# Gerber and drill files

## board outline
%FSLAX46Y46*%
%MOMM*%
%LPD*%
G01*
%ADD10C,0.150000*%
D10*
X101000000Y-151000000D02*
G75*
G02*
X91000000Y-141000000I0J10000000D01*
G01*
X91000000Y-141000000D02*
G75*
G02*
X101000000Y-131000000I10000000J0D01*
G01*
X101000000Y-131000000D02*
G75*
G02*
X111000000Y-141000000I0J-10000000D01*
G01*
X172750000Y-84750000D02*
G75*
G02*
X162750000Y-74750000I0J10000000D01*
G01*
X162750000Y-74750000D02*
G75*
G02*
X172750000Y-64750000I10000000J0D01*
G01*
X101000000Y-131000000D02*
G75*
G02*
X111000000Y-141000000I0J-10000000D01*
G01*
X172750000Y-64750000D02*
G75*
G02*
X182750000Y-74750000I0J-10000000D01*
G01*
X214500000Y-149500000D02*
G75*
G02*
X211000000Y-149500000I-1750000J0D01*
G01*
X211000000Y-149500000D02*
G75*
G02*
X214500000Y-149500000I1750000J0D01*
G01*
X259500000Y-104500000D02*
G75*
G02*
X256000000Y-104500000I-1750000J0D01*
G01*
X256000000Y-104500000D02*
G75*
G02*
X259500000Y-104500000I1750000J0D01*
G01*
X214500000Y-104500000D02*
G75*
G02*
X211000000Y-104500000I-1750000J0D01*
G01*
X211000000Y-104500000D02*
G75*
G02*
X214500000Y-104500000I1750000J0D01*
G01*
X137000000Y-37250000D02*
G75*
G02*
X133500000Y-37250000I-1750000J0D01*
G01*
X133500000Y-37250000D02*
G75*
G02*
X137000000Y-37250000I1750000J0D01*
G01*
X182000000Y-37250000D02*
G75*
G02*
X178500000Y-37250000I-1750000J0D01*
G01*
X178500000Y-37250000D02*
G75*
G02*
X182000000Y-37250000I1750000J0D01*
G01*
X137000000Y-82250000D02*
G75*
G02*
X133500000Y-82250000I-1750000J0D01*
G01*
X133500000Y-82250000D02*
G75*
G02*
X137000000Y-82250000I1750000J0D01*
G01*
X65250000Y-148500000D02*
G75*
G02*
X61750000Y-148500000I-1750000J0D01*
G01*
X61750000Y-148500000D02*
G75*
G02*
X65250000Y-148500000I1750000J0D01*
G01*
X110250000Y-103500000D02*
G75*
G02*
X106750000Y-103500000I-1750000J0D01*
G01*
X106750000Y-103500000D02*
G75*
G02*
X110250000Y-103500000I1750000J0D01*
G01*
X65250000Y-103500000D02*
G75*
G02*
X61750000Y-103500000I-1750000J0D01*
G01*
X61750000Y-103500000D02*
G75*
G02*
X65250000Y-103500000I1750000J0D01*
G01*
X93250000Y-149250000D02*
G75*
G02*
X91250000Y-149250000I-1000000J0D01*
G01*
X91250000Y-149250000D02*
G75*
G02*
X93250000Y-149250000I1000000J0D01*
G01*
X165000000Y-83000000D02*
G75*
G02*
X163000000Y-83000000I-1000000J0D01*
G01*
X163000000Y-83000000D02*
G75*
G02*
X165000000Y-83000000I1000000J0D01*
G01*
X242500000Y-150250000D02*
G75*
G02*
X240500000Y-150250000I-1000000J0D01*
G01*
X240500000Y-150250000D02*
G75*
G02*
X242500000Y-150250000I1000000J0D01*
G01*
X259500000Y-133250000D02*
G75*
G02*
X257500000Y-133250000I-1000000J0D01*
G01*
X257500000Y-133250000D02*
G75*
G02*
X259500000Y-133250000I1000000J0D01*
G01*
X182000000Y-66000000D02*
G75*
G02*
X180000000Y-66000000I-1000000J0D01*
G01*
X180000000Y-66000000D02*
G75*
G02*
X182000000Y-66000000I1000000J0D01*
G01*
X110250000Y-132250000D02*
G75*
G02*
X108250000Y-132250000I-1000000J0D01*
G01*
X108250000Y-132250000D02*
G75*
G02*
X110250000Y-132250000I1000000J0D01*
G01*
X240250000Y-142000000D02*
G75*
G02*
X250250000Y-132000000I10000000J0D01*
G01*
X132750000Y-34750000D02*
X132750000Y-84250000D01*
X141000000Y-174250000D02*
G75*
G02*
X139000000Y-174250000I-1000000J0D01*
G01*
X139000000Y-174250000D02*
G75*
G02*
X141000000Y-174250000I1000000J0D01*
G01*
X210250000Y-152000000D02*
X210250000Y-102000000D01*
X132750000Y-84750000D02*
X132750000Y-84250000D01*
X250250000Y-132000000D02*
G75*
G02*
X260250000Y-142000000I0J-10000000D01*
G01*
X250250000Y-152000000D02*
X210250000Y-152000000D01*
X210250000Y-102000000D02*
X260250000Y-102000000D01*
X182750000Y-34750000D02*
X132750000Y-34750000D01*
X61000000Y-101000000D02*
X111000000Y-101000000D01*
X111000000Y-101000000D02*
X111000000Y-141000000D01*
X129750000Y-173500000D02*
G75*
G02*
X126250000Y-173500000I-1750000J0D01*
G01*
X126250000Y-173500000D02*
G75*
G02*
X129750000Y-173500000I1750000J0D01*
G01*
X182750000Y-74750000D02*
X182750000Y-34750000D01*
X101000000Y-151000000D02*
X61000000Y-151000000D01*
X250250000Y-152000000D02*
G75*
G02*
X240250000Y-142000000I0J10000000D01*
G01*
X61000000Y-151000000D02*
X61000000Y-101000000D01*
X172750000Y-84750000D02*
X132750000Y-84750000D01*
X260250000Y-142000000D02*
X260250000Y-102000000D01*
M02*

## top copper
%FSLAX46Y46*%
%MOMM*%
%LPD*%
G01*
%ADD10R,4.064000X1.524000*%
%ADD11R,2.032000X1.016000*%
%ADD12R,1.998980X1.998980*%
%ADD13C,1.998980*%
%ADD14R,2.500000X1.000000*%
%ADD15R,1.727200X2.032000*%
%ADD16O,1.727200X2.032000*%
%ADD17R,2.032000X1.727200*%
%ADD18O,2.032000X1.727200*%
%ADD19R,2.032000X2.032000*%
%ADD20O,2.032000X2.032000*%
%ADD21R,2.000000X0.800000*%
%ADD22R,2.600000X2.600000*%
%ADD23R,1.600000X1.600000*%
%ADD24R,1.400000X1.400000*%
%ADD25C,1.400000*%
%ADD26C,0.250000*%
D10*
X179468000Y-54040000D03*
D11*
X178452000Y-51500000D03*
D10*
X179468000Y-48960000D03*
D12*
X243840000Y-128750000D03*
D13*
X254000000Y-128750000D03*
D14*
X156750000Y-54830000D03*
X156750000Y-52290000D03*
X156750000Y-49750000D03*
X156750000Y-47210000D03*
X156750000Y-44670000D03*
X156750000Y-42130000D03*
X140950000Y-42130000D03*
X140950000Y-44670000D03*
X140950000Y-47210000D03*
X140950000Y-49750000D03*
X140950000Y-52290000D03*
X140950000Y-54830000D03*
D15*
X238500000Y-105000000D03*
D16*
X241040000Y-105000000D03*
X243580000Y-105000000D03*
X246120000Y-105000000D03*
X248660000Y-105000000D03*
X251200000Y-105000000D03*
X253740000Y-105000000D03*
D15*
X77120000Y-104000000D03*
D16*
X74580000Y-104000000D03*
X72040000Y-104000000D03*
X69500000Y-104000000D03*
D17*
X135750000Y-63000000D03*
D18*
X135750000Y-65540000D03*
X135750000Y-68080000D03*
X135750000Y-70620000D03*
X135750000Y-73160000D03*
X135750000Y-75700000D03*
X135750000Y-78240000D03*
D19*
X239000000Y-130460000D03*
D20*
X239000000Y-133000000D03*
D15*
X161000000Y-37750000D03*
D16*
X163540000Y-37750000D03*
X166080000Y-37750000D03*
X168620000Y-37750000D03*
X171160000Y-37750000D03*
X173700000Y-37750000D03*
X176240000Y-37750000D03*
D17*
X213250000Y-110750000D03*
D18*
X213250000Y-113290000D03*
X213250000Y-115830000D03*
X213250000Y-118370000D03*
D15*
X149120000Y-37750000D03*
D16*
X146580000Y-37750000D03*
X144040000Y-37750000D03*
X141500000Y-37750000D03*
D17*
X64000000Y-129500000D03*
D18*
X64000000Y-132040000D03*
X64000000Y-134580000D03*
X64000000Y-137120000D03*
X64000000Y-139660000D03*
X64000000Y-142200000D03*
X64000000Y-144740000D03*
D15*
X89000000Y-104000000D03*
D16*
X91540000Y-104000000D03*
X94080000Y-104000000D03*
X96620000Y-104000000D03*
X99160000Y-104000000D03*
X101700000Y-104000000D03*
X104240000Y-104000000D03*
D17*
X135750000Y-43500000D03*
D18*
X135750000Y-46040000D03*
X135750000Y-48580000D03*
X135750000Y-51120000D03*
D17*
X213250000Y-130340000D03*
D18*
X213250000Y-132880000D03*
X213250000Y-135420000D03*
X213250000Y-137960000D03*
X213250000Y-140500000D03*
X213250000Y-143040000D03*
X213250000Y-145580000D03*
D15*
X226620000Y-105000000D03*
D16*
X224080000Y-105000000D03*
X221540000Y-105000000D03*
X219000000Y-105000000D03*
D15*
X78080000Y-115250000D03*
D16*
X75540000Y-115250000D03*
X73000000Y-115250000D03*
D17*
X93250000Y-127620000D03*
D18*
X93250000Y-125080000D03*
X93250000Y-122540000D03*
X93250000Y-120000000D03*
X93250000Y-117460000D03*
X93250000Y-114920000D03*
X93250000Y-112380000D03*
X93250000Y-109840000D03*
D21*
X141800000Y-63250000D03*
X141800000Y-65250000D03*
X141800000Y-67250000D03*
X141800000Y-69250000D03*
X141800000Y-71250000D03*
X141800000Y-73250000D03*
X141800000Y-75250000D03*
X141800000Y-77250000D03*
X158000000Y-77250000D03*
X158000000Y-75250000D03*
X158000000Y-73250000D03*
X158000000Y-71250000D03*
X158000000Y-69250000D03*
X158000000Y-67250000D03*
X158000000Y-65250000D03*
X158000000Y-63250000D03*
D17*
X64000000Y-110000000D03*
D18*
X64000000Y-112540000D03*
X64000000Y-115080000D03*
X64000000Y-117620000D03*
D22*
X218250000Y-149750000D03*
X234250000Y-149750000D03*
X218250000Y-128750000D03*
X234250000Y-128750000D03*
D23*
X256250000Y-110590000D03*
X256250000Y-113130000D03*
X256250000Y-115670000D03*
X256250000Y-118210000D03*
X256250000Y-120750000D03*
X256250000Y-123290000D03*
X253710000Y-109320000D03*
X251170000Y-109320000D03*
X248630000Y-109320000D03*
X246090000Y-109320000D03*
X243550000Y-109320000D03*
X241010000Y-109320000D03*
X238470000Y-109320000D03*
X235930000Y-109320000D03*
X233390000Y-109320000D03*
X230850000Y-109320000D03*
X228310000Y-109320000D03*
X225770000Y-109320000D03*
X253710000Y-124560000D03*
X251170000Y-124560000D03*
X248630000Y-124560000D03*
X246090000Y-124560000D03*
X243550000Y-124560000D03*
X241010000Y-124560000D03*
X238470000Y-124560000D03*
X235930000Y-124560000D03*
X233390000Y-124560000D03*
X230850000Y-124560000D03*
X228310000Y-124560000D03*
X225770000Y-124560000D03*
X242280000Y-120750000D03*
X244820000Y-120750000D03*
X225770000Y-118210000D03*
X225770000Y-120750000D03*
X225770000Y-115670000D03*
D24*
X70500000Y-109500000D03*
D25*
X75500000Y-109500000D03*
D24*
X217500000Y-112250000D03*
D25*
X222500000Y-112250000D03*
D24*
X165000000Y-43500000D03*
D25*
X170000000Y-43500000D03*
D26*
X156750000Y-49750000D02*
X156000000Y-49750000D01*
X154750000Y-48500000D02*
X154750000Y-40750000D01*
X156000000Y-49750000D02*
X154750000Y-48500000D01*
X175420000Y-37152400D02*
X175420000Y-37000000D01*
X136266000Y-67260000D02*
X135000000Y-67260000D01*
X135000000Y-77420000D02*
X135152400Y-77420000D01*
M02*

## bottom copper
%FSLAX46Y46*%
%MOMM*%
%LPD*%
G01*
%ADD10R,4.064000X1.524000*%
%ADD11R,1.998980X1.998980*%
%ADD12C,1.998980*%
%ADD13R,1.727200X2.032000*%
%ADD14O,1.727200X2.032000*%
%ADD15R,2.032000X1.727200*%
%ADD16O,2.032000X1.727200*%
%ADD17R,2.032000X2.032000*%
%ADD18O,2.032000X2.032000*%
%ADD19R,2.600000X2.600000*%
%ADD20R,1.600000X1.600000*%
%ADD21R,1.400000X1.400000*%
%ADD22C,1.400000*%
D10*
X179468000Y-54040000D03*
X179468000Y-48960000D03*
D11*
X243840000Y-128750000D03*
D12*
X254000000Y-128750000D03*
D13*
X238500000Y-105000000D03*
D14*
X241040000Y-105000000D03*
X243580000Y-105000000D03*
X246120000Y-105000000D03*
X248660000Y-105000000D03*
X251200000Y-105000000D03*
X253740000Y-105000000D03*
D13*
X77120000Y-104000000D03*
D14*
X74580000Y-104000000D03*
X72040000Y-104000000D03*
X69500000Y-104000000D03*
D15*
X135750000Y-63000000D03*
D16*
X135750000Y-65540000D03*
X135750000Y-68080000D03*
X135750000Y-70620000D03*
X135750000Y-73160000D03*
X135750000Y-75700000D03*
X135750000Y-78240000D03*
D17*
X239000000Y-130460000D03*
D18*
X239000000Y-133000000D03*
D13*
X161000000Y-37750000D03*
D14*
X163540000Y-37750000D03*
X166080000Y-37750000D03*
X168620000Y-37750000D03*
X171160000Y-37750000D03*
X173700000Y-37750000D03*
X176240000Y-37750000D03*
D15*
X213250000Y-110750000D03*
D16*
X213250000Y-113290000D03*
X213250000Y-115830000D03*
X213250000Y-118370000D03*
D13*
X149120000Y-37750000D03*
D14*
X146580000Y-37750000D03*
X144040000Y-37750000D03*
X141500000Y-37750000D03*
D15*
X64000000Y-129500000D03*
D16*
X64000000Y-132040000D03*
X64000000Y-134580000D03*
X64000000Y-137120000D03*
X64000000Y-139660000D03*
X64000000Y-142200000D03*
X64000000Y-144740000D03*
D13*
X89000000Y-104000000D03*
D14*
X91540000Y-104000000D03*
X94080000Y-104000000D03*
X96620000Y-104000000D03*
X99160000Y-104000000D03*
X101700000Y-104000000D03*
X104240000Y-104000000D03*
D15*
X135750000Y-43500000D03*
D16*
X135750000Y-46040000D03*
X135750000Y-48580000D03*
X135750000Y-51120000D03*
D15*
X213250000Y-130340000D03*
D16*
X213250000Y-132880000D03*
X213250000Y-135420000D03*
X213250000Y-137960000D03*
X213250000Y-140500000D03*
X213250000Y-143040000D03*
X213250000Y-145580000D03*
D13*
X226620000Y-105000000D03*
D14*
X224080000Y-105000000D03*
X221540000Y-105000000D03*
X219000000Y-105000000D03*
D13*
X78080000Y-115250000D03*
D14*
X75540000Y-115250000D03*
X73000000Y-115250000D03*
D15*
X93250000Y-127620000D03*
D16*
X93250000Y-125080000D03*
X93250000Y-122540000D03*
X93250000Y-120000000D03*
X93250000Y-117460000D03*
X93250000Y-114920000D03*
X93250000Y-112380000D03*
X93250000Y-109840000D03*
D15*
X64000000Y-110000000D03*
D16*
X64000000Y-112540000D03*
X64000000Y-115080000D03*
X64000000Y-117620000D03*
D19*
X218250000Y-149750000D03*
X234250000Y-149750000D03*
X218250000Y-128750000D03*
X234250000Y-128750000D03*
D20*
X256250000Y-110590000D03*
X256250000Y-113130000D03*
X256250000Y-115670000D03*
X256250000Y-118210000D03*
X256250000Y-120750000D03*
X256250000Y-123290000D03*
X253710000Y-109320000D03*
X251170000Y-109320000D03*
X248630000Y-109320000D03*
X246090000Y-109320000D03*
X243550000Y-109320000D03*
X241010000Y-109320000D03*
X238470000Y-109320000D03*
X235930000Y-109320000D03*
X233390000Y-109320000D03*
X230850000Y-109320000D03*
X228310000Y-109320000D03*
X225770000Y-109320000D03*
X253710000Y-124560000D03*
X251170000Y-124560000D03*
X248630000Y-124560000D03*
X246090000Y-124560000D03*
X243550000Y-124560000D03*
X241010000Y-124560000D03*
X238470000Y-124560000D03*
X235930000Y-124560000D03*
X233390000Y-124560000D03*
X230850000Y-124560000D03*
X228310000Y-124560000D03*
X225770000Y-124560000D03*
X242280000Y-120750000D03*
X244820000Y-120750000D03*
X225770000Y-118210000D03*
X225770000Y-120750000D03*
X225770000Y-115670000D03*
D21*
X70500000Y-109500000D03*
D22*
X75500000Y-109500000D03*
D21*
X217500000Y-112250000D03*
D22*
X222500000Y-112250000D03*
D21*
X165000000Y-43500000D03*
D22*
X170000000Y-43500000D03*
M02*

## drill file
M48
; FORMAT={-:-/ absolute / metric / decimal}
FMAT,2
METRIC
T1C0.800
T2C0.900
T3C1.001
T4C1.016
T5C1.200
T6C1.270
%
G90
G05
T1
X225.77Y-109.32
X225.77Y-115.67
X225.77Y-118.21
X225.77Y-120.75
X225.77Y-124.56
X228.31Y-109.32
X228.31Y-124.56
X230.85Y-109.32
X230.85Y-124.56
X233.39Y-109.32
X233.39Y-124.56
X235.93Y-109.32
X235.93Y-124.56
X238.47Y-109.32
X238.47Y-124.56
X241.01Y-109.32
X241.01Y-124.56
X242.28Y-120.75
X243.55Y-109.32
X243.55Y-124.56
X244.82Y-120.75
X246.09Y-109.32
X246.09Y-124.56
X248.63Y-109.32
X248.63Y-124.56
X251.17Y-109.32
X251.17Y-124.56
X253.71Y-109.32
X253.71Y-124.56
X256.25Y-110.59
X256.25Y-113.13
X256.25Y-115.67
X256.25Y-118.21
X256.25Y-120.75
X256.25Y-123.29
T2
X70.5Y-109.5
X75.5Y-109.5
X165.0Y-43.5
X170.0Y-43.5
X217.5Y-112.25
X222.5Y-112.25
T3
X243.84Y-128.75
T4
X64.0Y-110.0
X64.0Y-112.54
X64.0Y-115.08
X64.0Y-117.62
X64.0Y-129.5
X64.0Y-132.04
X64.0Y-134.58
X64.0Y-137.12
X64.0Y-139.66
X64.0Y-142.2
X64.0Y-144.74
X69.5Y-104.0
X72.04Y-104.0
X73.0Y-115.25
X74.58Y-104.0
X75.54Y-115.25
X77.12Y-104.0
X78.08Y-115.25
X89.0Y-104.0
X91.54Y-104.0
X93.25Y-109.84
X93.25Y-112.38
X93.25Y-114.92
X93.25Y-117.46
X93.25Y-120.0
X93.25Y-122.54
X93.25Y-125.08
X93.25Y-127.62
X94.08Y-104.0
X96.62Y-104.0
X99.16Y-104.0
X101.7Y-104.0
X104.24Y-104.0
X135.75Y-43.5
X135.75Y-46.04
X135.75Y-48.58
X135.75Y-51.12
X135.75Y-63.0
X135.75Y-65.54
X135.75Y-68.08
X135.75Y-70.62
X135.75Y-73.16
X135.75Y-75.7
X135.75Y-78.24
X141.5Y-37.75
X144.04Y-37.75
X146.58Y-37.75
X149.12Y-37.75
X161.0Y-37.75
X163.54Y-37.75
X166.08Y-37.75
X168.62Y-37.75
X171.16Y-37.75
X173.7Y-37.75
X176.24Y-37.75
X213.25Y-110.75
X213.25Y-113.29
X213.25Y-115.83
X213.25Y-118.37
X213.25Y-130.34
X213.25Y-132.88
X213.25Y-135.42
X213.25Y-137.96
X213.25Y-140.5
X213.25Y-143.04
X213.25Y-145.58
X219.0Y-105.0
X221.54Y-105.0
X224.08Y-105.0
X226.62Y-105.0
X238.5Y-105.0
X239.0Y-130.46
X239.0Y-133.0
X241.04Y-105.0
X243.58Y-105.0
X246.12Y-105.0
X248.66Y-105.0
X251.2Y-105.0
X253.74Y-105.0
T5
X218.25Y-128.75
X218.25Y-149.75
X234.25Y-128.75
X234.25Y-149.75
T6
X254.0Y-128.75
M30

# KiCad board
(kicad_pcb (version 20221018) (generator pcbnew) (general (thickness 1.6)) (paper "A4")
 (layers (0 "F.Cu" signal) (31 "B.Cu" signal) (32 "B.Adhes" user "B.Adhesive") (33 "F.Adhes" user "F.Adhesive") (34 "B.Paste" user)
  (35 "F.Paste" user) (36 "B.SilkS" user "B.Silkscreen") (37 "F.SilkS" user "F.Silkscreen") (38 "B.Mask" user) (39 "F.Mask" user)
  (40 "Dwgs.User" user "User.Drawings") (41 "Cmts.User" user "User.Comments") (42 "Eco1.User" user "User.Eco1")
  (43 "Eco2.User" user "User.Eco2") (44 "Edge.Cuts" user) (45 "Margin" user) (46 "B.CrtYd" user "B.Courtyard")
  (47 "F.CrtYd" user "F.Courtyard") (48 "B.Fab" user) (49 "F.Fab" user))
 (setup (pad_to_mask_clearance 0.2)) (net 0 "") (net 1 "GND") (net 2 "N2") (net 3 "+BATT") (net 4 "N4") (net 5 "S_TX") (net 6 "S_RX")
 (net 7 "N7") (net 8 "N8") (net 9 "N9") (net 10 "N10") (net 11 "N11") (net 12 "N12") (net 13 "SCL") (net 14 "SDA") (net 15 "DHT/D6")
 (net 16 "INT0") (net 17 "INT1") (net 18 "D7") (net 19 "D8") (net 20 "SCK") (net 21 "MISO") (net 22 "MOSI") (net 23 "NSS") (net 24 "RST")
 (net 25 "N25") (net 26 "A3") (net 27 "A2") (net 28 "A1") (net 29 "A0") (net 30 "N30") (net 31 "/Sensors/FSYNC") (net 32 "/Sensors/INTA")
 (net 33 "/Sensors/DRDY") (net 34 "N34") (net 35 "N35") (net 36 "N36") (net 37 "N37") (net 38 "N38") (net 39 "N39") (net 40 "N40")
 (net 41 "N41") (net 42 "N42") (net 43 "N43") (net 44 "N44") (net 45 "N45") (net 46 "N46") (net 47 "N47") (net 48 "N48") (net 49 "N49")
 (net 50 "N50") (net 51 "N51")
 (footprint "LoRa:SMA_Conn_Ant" (layer "F.Cu") (at 181.5 51.5 180)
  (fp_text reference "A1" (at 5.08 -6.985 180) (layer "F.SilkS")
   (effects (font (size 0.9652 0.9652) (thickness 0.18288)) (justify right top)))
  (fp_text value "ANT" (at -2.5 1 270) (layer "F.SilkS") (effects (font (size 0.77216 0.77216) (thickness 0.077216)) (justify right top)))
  (pad "" smd rect (at 2.032 -2.54 270) (size 1.524 4.064) (layers "B.Cu" "B.Paste" "B.Mask"))
  (pad "" smd rect (at 2.032 2.54 270) (size 1.524 4.064) (layers "B.Cu" "B.Paste" "B.Mask"))
  (pad "1" smd rect (at 2.032 -2.54 270) (size 1.524 4.064) (layers "F.Cu" "F.Paste" "F.Mask") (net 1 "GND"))
  (pad "2" smd rect (at 3.048 0 270) (size 1.016 2.032) (layers "F.Cu" "F.Paste" "F.Mask") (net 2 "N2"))
  (pad "3" smd rect (at 2.032 2.54 270) (size 1.524 4.064) (layers "F.Cu" "F.Paste" "F.Mask") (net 1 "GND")))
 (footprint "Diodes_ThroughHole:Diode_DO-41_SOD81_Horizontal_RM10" (layer "F.Cu") (at 243.84 128.75254)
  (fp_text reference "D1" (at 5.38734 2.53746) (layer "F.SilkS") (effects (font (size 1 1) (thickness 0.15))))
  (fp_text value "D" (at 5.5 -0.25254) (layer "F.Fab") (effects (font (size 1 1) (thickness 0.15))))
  (pad "1" thru_hole rect (at 0 -0.00254 180) (size 1.99898 1.99898) (drill 1.00076) (layers "*.Cu" "*.Mask" "F.SilkS") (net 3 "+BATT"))
  (pad "2" thru_hole circle (at 10.16 -0.00254 180) (size 1.99898 1.99898) (drill 1.27) (layers "*.Cu" "*.Mask" "F.SilkS") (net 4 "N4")))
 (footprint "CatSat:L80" (layer "F.Cu") (at 148.883668 49.118506 180) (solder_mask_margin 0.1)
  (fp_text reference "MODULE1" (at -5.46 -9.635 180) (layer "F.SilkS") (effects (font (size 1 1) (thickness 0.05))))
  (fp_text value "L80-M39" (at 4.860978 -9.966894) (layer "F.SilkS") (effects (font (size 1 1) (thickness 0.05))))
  (pad "1" smd rect (at -7.866332 -5.711494) (size 2.5 1) (layers "F.Cu" "F.Paste" "F.Mask") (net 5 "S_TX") (solder_mask_margin 0.2))
  (pad "2" smd rect (at -7.866332 -3.171494) (size 2.5 1) (layers "F.Cu" "F.Paste" "F.Mask") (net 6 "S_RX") (solder_mask_margin 0.2))
  (pad "3" smd rect (at -7.866332 -0.631494) (size 2.5 1) (layers "F.Cu" "F.Paste" "F.Mask") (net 1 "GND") (solder_mask_margin 0.2))
  (pad "4" smd rect (at -7.866332 1.908506) (size 2.5 1) (layers "F.Cu" "F.Paste" "F.Mask") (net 3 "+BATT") (solder_mask_margin 0.2))
  (pad "5" smd rect (at -7.866332 4.448506) (size 2.5 1) (layers "F.Cu" "F.Paste" "F.Mask") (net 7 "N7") (solder_mask_margin 0.2))
  (pad "6" smd rect (at -7.866332 6.988506) (size 2.5 1) (layers "F.Cu" "F.Paste" "F.Mask") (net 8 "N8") (solder_mask_margin 0.2))
  (pad "7" smd rect (at 7.933668 6.988506 180) (size 2.5 1) (layers "F.Cu" "F.Paste" "F.Mask") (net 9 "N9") (solder_mask_margin 0.2))
  (pad "8" smd rect (at 7.933668 4.448506 180) (size 2.5 1) (layers "F.Cu" "F.Paste" "F.Mask") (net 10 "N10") (solder_mask_margin 0.2))
  (pad "9" smd rect (at 7.933668 1.908506 180) (size 2.5 1) (layers "F.Cu" "F.Paste" "F.Mask") (solder_mask_margin 0.2))
  (pad "10" smd rect (at 7.933668 -0.631494 180) (size 2.5 1) (layers "F.Cu" "F.Paste" "F.Mask") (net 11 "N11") (solder_mask_margin 0.2))
  (pad "11" smd rect (at 7.933668 -3.171494 180) (size 2.5 1) (layers "F.Cu" "F.Paste" "F.Mask") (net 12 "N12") (solder_mask_margin 0.2))
  (pad "12" smd rect (at 7.933668 -5.711494) (size 2.5 1) (layers "F.Cu" "F.Paste" "F.Mask") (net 1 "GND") (solder_mask_margin 0.2)))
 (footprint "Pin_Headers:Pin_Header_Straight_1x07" (layer "F.Cu") (at 238.5 105 90)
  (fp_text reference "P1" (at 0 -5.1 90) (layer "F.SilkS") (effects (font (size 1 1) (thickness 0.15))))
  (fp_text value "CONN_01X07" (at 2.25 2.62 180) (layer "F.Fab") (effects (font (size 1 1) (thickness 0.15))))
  (pad "1" thru_hole rect (at 0 0 90) (size 2.032 1.7272) (drill 1.016) (layers "*.Cu" "*.Mask" "F.SilkS") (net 1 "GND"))
  (pad "2" thru_hole oval (at 0 2.54 90) (size 2.032 1.7272) (drill 1.016) (layers "*.Cu" "*.Mask" "F.SilkS") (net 3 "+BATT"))
  (pad "3" thru_hole oval (at 0 5.08 90) (size 2.032 1.7272) (drill 1.016) (layers "*.Cu" "*.Mask" "F.SilkS") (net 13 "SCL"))
  (pad "4" thru_hole oval (at 0 7.62 90) (size 2.032 1.7272) (drill 1.016) (layers "*.Cu" "*.Mask" "F.SilkS") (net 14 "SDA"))
  (pad "5" thru_hole oval (at 0 10.16 90) (size 2.032 1.7272) (drill 1.016) (layers "*.Cu" "*.Mask" "F.SilkS") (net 6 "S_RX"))
  (pad "6" thru_hole oval (at 0 12.7 90) (size 2.032 1.7272) (drill 1.016) (layers "*.Cu" "*.Mask" "F.SilkS") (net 5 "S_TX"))
  (pad "7" thru_hole oval (at 0 15.24 90) (size 2.032 1.7272) (drill 1.016) (layers "*.Cu" "*.Mask" "F.SilkS") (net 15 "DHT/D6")))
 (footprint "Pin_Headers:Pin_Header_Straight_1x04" (layer "F.Cu") (at 77.12 104 -90)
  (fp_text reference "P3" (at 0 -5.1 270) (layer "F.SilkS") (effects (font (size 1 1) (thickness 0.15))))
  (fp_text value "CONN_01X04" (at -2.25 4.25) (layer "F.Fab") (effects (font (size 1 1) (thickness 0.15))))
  (pad "1" thru_hole rect (at 0 0 270) (size 2.032 1.7272) (drill 1.016) (layers "*.Cu" "*.Mask" "F.SilkS") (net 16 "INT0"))
  (pad "2" thru_hole oval (at 0 2.54 270) (size 2.032 1.7272) (drill 1.016) (layers "*.Cu" "*.Mask" "F.SilkS") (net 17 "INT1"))
  (pad "3" thru_hole oval (at 0 5.08 270) (size 2.032 1.7272) (drill 1.016) (layers "*.Cu" "*.Mask" "F.SilkS") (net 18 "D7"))
  (pad "4" thru_hole oval (at 0 7.62 270) (size 2.032 1.7272) (drill 1.016) (layers "*.Cu" "*.Mask" "F.SilkS") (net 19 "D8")))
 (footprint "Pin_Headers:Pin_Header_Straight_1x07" (layer "F.Cu") (at 135.75 63)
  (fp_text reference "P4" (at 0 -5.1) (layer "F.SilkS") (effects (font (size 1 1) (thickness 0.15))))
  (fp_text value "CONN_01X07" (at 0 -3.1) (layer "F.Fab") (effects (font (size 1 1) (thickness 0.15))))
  (pad "1" thru_hole rect (at 0 0) (size 2.032 1.7272) (drill 1.016) (layers "*.Cu" "*.Mask" "F.SilkS") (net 3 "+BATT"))
  (pad "2" thru_hole oval (at 0 2.54) (size 2.032 1.7272) (drill 1.016) (layers "*.Cu" "*.Mask" "F.SilkS") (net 1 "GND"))
  (pad "3" thru_hole oval (at 0 5.08) (size 2.032 1.7272) (drill 1.016) (layers "*.Cu" "*.Mask" "F.SilkS") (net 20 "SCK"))
  (pad "4" thru_hole oval (at 0 7.62) (size 2.032 1.7272) (drill 1.016) (layers "*.Cu" "*.Mask" "F.SilkS") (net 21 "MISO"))
  (pad "5" thru_hole oval (at 0 10.16) (size 2.032 1.7272) (drill 1.016) (layers "*.Cu" "*.Mask" "F.SilkS") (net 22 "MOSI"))
  (pad "6" thru_hole oval (at 0 12.7) (size 2.032 1.7272) (drill 1.016) (layers "*.Cu" "*.Mask" "F.SilkS") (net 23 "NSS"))
  (pad "7" thru_hole oval (at 0 15.24) (size 2.032 1.7272) (drill 1.016) (layers "*.Cu" "*.Mask" "F.SilkS") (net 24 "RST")))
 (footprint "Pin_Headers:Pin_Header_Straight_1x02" (layer "F.Cu") (at 239 130.46)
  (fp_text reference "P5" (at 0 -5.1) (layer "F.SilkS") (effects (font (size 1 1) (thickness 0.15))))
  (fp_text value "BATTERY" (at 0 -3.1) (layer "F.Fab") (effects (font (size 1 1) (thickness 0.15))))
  (pad "1" thru_hole rect (at 0 0) (size 2.032 2.032) (drill 1.016) (layers "*.Cu" "*.Mask" "F.SilkS") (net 4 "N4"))
  (pad "2" thru_hole oval (at 0 2.54) (size 2.032 2.032) (drill 1.016) (layers "*.Cu" "*.Mask" "F.SilkS") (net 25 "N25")))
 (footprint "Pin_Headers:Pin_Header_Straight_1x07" (layer "F.Cu") (at 161 37.75 90)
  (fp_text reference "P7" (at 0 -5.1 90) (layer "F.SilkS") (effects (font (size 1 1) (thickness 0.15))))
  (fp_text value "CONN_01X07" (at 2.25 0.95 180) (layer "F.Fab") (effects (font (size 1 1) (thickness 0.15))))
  (pad "1" thru_hole rect (at 0 0 90) (size 2.032 1.7272) (drill 1.016) (layers "*.Cu" "*.Mask" "F.SilkS") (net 1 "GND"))
  (pad "2" thru_hole oval (at 0 2.54 90) (size 2.032 1.7272) (drill 1.016) (layers "*.Cu" "*.Mask" "F.SilkS") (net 3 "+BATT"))
  (pad "3" thru_hole oval (at 0 5.08 90) (size 2.032 1.7272) (drill 1.016) (layers "*.Cu" "*.Mask" "F.SilkS") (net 13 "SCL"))
  (pad "4" thru_hole oval (at 0 7.62 90) (size 2.032 1.7272) (drill 1.016) (layers "*.Cu" "*.Mask" "F.SilkS") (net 14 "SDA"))
  (pad "5" thru_hole oval (at 0 10.16 90) (size 2.032 1.7272) (drill 1.016) (layers "*.Cu" "*.Mask" "F.SilkS") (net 6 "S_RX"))
  (pad "6" thru_hole oval (at 0 12.7 90) (size 2.032 1.7272) (drill 1.016) (layers "*.Cu" "*.Mask" "F.SilkS") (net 5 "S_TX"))
  (pad "7" thru_hole oval (at 0 15.24 90) (size 2.032 1.7272) (drill 1.016) (layers "*.Cu" "*.Mask" "F.SilkS") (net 15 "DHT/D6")))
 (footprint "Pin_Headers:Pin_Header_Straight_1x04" (layer "F.Cu") (at 213.25 110.75)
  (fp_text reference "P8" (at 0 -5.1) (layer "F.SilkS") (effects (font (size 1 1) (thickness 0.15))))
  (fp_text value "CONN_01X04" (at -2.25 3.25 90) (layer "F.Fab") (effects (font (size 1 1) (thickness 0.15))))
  (pad "1" thru_hole rect (at 0 0) (size 2.032 1.7272) (drill 1.016) (layers "*.Cu" "*.Mask" "F.SilkS") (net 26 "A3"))
  (pad "2" thru_hole oval (at 0 2.54) (size 2.032 1.7272) (drill 1.016) (layers "*.Cu" "*.Mask" "F.SilkS") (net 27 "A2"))
  (pad "3" thru_hole oval (at 0 5.08) (size 2.032 1.7272) (drill 1.016) (layers "*.Cu" "*.Mask" "F.SilkS") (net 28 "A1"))
  (pad "4" thru_hole oval (at 0 7.62) (size 2.032 1.7272) (drill 1.016) (layers "*.Cu" "*.Mask" "F.SilkS") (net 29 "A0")))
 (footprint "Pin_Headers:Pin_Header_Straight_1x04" (layer "F.Cu") (at 149.12 37.75 -90)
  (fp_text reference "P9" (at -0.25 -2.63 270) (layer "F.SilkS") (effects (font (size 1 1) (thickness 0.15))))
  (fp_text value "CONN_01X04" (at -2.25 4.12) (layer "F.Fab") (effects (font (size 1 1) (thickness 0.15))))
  (pad "1" thru_hole rect (at 0 0 270) (size 2.032 1.7272) (drill 1.016) (layers "*.Cu" "*.Mask" "F.SilkS") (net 16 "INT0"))
  (pad "2" thru_hole oval (at 0 2.54 270) (size 2.032 1.7272) (drill 1.016) (layers "*.Cu" "*.Mask" "F.SilkS") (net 17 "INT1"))
  (pad "3" thru_hole oval (at 0 5.08 270) (size 2.032 1.7272) (drill 1.016) (layers "*.Cu" "*.Mask" "F.SilkS") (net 18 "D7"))
  (pad "4" thru_hole oval (at 0 7.62 270) (size 2.032 1.7272) (drill 1.016) (layers "*.Cu" "*.Mask" "F.SilkS") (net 19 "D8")))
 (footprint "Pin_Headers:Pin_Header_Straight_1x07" (layer "F.Cu") (at 64 129.5)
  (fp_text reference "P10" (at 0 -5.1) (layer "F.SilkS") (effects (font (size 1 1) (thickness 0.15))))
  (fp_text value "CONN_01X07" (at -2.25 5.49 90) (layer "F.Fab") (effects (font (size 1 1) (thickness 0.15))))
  (pad "1" thru_hole rect (at 0 0) (size 2.032 1.7272) (drill 1.016) (layers "*.Cu" "*.Mask" "F.SilkS") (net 3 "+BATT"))
  (pad "2" thru_hole oval (at 0 2.54) (size 2.032 1.7272) (drill 1.016) (layers "*.Cu" "*.Mask" "F.SilkS") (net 1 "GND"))
  (pad "3" thru_hole oval (at 0 5.08) (size 2.032 1.7272) (drill 1.016) (layers "*.Cu" "*.Mask" "F.SilkS") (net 20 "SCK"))
  (pad "4" thru_hole oval (at 0 7.62) (size 2.032 1.7272) (drill 1.016) (layers "*.Cu" "*.Mask" "F.SilkS") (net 21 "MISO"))
  (pad "5" thru_hole oval (at 0 10.16) (size 2.032 1.7272) (drill 1.016) (layers "*.Cu" "*.Mask" "F.SilkS") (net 22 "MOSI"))
  (pad "6" thru_hole oval (at 0 12.7) (size 2.032 1.7272) (drill 1.016) (layers "*.Cu" "*.Mask" "F.SilkS") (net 23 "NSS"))
  (pad "7" thru_hole oval (at 0 15.24) (size 2.032 1.7272) (drill 1.016) (layers "*.Cu" "*.Mask" "F.SilkS") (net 24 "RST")))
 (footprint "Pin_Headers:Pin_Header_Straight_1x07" (layer "F.Cu") (at 89 104 90)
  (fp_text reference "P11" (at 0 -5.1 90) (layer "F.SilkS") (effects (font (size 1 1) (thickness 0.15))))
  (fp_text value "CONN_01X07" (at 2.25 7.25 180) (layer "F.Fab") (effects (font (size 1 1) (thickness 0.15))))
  (pad "1" thru_hole rect (at 0 0 90) (size 2.032 1.7272) (drill 1.016) (layers "*.Cu" "*.Mask" "F.SilkS") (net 1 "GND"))
  (pad "2" thru_hole oval (at 0 2.54 90) (size 2.032 1.7272) (drill 1.016) (layers "*.Cu" "*.Mask" "F.SilkS") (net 3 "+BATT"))
  (pad "3" thru_hole oval (at 0 5.08 90) (size 2.032 1.7272) (drill 1.016) (layers "*.Cu" "*.Mask" "F.SilkS") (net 13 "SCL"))
  (pad "4" thru_hole oval (at 0 7.62 90) (size 2.032 1.7272) (drill 1.016) (layers "*.Cu" "*.Mask" "F.SilkS") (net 14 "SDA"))
  (pad "5" thru_hole oval (at 0 10.16 90) (size 2.032 1.7272) (drill 1.016) (layers "*.Cu" "*.Mask" "F.SilkS") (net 6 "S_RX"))
  (pad "6" thru_hole oval (at 0 12.7 90) (size 2.032 1.7272) (drill 1.016) (layers "*.Cu" "*.Mask" "F.SilkS") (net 5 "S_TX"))
  (pad "7" thru_hole oval (at 0 15.24 90) (size 2.032 1.7272) (drill 1.016) (layers "*.Cu" "*.Mask" "F.SilkS") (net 15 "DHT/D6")))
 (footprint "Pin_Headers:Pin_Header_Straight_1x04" (layer "F.Cu") (at 135.75 43.5)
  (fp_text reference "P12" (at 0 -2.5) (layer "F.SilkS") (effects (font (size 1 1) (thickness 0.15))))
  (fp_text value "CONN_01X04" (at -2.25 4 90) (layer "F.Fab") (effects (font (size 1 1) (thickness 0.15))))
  (pad "1" thru_hole rect (at 0 0) (size 2.032 1.7272) (drill 1.016) (layers "*.Cu" "*.Mask" "F.SilkS") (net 26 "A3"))
  (pad "2" thru_hole oval (at 0 2.54) (size 2.032 1.7272) (drill 1.016) (layers "*.Cu" "*.Mask" "F.SilkS") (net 27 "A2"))
  (pad "3" thru_hole oval (at 0 5.08) (size 2.032 1.7272) (drill 1.016) (layers "*.Cu" "*.Mask" "F.SilkS") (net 28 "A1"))
  (pad "4" thru_hole oval (at 0 7.62) (size 2.032 1.7272) (drill 1.016) (layers "*.Cu" "*.Mask" "F.SilkS") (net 29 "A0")))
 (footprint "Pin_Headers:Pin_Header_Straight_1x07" (layer "F.Cu") (at 213.25 130.34)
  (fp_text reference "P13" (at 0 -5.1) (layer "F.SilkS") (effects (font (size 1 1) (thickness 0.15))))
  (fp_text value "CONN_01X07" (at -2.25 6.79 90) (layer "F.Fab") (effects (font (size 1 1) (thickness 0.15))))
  (pad "1" thru_hole rect (at 0 0) (size 2.032 1.7272) (drill 1.016) (layers "*.Cu" "*.Mask" "F.SilkS") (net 3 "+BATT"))
  (pad "2" thru_hole oval (at 0 2.54) (size 2.032 1.7272) (drill 1.016) (layers "*.Cu" "*.Mask" "F.SilkS") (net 1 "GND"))
  (pad "3" thru_hole oval (at 0 5.08) (size 2.032 1.7272) (drill 1.016) (layers "*.Cu" "*.Mask" "F.SilkS") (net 20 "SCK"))
  (pad "4" thru_hole oval (at 0 7.62) (size 2.032 1.7272) (drill 1.016) (layers "*.Cu" "*.Mask" "F.SilkS") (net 21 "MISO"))
  (pad "5" thru_hole oval (at 0 10.16) (size 2.032 1.7272) (drill 1.016) (layers "*.Cu" "*.Mask" "F.SilkS") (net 22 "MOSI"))
  (pad "6" thru_hole oval (at 0 12.7) (size 2.032 1.7272) (drill 1.016) (layers "*.Cu" "*.Mask" "F.SilkS") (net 23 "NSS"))
  (pad "7" thru_hole oval (at 0 15.24) (size 2.032 1.7272) (drill 1.016) (layers "*.Cu" "*.Mask" "F.SilkS") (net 24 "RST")))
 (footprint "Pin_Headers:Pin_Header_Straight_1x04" (layer "F.Cu") (at 226.62 105 -90)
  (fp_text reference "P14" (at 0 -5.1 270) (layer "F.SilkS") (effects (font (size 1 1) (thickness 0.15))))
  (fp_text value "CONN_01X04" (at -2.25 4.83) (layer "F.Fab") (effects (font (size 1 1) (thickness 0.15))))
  (pad "1" thru_hole rect (at 0 0 270) (size 2.032 1.7272) (drill 1.016) (layers "*.Cu" "*.Mask" "F.SilkS") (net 16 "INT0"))
  (pad "2" thru_hole oval (at 0 2.54 270) (size 2.032 1.7272) (drill 1.016) (layers "*.Cu" "*.Mask" "F.SilkS") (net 17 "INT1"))
  (pad "3" thru_hole oval (at 0 5.08 270) (size 2.032 1.7272) (drill 1.016) (layers "*.Cu" "*.Mask" "F.SilkS") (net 18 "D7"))
  (pad "4" thru_hole oval (at 0 7.62 270) (size 2.032 1.7272) (drill 1.016) (layers "*.Cu" "*.Mask" "F.SilkS") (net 19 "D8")))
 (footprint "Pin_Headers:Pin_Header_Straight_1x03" (layer "F.Cu") (at 78.08 115.25 -90)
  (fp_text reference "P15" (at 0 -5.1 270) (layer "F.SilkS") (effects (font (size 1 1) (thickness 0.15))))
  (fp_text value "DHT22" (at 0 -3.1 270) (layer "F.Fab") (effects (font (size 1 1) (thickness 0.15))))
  (pad "1" thru_hole rect (at 0 0 270) (size 2.032 1.7272) (drill 1.016) (layers "*.Cu" "*.Mask" "F.SilkS") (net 15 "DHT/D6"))
  (pad "2" thru_hole oval (at 0 2.54 270) (size 2.032 1.7272) (drill 1.016) (layers "*.Cu" "*.Mask" "F.SilkS") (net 3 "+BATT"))
  (pad "3" thru_hole oval (at 0 5.08 270) (size 2.032 1.7272) (drill 1.016) (layers "*.Cu" "*.Mask" "F.SilkS") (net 1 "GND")))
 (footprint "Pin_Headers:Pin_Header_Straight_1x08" (layer "F.Cu") (at 93.25 127.62 180)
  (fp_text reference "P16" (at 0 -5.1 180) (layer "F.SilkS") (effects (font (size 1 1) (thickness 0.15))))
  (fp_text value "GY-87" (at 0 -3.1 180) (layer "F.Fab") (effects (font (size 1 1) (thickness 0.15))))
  (pad "1" thru_hole rect (at 0 0 180) (size 2.032 1.7272) (drill 1.016) (layers "*.Cu" "*.Mask" "F.SilkS") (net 3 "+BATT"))
  (pad "2" thru_hole oval (at 0 2.54 180) (size 2.032 1.7272) (drill 1.016) (layers "*.Cu" "*.Mask" "F.SilkS") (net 1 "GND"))
  (pad "3" thru_hole oval (at 0 5.08 180) (size 2.032 1.7272) (drill 1.016) (layers "*.Cu" "*.Mask" "F.SilkS") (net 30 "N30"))
  (pad "4" thru_hole oval (at 0 7.62 180) (size 2.032 1.7272) (drill 1.016) (layers "*.Cu" "*.Mask" "F.SilkS") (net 13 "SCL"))
  (pad "5" thru_hole oval (at 0 10.16 180) (size 2.032 1.7272) (drill 1.016) (layers "*.Cu" "*.Mask" "F.SilkS") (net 14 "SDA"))
  (pad "6" thru_hole oval (at 0 12.7 180) (size 2.032 1.7272) (drill 1.016) (layers "*.Cu" "*.Mask" "F.SilkS") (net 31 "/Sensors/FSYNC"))
  (pad "7" thru_hole oval (at 0 15.24 180) (size 2.032 1.7272) (drill 1.016) (layers "*.Cu" "*.Mask" "F.SilkS") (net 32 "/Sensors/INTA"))
  (pad "8" thru_hole oval (at 0 17.78 180) (size 2.032 1.7272) (drill 1.016) (layers "*.Cu" "*.Mask" "F.SilkS") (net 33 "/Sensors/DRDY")))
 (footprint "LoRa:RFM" (layer "F.Cu") (at 149.9 70.25)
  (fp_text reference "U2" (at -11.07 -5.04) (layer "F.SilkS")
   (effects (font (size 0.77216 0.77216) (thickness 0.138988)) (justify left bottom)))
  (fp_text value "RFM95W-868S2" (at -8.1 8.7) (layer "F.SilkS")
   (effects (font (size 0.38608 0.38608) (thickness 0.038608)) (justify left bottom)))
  (pad "1" smd rect (at -8.1 -7) (size 2 0.8) (layers "F.Cu" "F.Paste" "F.Mask") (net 1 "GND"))
  (pad "2" smd rect (at -8.1 -5) (size 2 0.8) (layers "F.Cu" "F.Paste" "F.Mask") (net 21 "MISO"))
  (pad "3" smd rect (at -8.1 -3) (size 2 0.8) (layers "F.Cu" "F.Paste" "F.Mask") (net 22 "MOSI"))
  (pad "4" smd rect (at -8.1 -1) (size 2 0.8) (layers "F.Cu" "F.Paste" "F.Mask") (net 20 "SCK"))
  (pad "5" smd rect (at -8.1 1) (size 2 0.8) (layers "F.Cu" "F.Paste" "F.Mask") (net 23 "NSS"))
  (pad "6" smd rect (at -8.1 3) (size 2 0.8) (layers "F.Cu" "F.Paste" "F.Mask") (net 24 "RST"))
  (pad "7" smd rect (at -8.1 5) (size 2 0.8) (layers "F.Cu" "F.Paste" "F.Mask") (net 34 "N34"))
  (pad "8" smd rect (at -8.1 7 180) (size 2 0.8) (layers "F.Cu" "F.Paste" "F.Mask") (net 1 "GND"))
  (pad "9" smd rect (at 8.1 7 180) (size 2 0.8) (layers "F.Cu" "F.Paste" "F.Mask") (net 2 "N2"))
  (pad "10" smd rect (at 8.1 5 180) (size 2 0.8) (layers "F.Cu" "F.Paste" "F.Mask") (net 1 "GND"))
  (pad "11" smd rect (at 8.1 3 180) (size 2 0.8) (layers "F.Cu" "F.Paste" "F.Mask") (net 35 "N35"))
  (pad "12" smd rect (at 8.1 1 180) (size 2 0.8) (layers "F.Cu" "F.Paste" "F.Mask") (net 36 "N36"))
  (pad "13" smd rect (at 8.1 -1 180) (size 2 0.8) (layers "F.Cu" "F.Paste" "F.Mask") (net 3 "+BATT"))
  (pad "14" smd rect (at 8.1 -3 180) (size 2 0.8) (layers "F.Cu" "F.Paste" "F.Mask") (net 16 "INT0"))
  (pad "15" smd rect (at 8.1 -5 180) (size 2 0.8) (layers "F.Cu" "F.Paste" "F.Mask") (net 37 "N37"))
  (pad "16" smd rect (at 8.1 -7 180) (size 2 0.8) (layers "F.Cu" "F.Paste" "F.Mask") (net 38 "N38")))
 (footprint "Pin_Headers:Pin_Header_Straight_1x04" (layer "F.Cu") (at 64 110)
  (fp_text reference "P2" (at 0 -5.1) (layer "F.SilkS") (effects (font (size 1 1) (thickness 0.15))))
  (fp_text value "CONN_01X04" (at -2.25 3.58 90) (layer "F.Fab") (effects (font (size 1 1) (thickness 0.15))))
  (pad "1" thru_hole rect (at 0 0) (size 2.032 1.7272) (drill 1.016) (layers "*.Cu" "*.Mask" "F.SilkS") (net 26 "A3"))
  (pad "2" thru_hole oval (at 0 2.54) (size 2.032 1.7272) (drill 1.016) (layers "*.Cu" "*.Mask" "F.SilkS") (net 27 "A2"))
  (pad "3" thru_hole oval (at 0 5.08) (size 2.032 1.7272) (drill 1.016) (layers "*.Cu" "*.Mask" "F.SilkS") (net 28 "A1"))
  (pad "4" thru_hole oval (at 0 7.62) (size 2.032 1.7272) (drill 1.016) (layers "*.Cu" "*.Mask" "F.SilkS") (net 29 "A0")))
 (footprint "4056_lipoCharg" (layer "F.Cu") (at 215.5 125.5)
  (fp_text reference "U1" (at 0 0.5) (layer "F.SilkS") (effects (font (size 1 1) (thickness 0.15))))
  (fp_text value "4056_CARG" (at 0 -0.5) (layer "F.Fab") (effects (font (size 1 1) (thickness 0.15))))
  (pad "1" thru_hole rect (at 2.75 24.25) (size 2.6 2.6) (drill 1.2) (layers "*.Cu" "*.Mask" "F.SilkS") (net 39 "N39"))
  (pad "2" thru_hole rect (at 18.75 24.25) (size 2.6 2.6) (drill 1.2) (layers "*.Cu" "*.Mask" "F.SilkS") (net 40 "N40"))
  (pad "3" thru_hole rect (at 2.75 3.25) (size 2.6 2.6) (drill 1.2) (layers "*.Cu" "*.Mask" "F.SilkS") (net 4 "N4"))
  (pad "4" thru_hole rect (at 18.75 3.25) (size 2.6 2.6) (drill 1.2) (layers "*.Cu" "*.Mask" "F.SilkS") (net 25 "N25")))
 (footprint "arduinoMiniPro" (layer "F.Cu") (at 247.36 114.4 -90)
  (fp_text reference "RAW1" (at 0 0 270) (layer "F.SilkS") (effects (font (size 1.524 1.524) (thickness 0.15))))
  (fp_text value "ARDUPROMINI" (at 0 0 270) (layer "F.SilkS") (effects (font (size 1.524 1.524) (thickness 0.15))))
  (pad "1" thru_hole rect (at -3.81 -8.89) (size 1.6 1.6) (drill 0.8) (layers "*.Cu" "*.Mask") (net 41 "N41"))
  (pad "2" thru_hole rect (at -1.27 -8.89) (size 1.6 1.6) (drill 0.8) (layers "*.Cu" "*.Mask") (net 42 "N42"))
  (pad "3" thru_hole rect (at 1.27 -8.89) (size 1.6 1.6) (drill 0.8) (layers "*.Cu" "*.Mask") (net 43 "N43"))
  (pad "4" thru_hole rect (at 3.81 -8.89) (size 1.6 1.6) (drill 0.8) (layers "*.Cu" "*.Mask") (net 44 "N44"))
  (pad "5" thru_hole rect (at 6.35 -8.89) (size 1.6 1.6) (drill 0.8) (layers "*.Cu" "*.Mask") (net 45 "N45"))
  (pad "6" thru_hole rect (at 8.89 -8.89) (size 1.6 1.6) (drill 0.8) (layers "*.Cu" "*.Mask") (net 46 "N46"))
  (pad "7" thru_hole rect (at -5.08 -6.35 90) (size 1.6 1.6) (drill 0.8) (layers "*.Cu" "*.Mask") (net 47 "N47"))
  (pad "8" thru_hole rect (at -5.08 -3.81 90) (size 1.6 1.6) (drill 0.8) (layers "*.Cu" "*.Mask") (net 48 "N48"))
  (pad "9" thru_hole rect (at -5.08 -1.27 90) (size 1.6 1.6) (drill 0.8) (layers "*.Cu" "*.Mask") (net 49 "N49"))
  (pad "10" thru_hole rect (at -5.08 1.27 90) (size 1.6 1.6) (drill 0.8) (layers "*.Cu" "*.Mask") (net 1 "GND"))
  (pad "11" thru_hole rect (at -5.08 3.81 90) (size 1.6 1.6) (drill 0.8) (layers "*.Cu" "*.Mask") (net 16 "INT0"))
  (pad "12" thru_hole rect (at -5.08 6.35 90) (size 1.6 1.6) (drill 0.8) (layers "*.Cu" "*.Mask") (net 17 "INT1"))
  (pad "13" thru_hole rect (at -5.08 8.89 90) (size 1.6 1.6) (drill 0.8) (layers "*.Cu" "*.Mask") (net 5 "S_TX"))
  (pad "14" thru_hole rect (at -5.08 11.43 90) (size 1.6 1.6) (drill 0.8) (layers "*.Cu" "*.Mask") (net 6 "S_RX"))
  (pad "15" thru_hole rect (at -5.08 13.97 90) (size 1.6 1.6) (drill 0.8) (layers "*.Cu" "*.Mask") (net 15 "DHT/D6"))
  (pad "16" thru_hole rect (at -5.08 16.51 90) (size 1.6 1.6) (drill 0.8) (layers "*.Cu" "*.Mask") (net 18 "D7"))
  (pad "17" thru_hole rect (at -5.08 19.05 90) (size 1.6 1.6) (drill 0.8) (layers "*.Cu" "*.Mask") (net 19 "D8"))
  (pad "18" thru_hole rect (at -5.08 21.59 90) (size 1.6 1.6) (drill 0.8) (layers "*.Cu" "*.Mask") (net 24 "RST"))
  (pad "19" thru_hole rect (at 10.16 -6.35 90) (size 1.6 1.6) (drill 0.8) (layers "*.Cu" "*.Mask") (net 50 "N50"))
  (pad "20" thru_hole rect (at 10.16 -3.81 90) (size 1.6 1.6) (drill 0.8) (layers "*.Cu" "*.Mask") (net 1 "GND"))
  (pad "21" thru_hole rect (at 10.16 -1.27 90) (size 1.6 1.6) (drill 0.8) (layers "*.Cu" "*.Mask") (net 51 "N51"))
  (pad "22" thru_hole rect (at 10.16 1.27 90) (size 1.6 1.6) (drill 0.8) (layers "*.Cu" "*.Mask") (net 3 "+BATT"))
  (pad "23" thru_hole rect (at 10.16 3.81 90) (size 1.6 1.6) (drill 0.8) (layers "*.Cu" "*.Mask") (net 26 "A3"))
  (pad "24" thru_hole rect (at 10.16 6.35 90) (size 1.6 1.6) (drill 0.8) (layers "*.Cu" "*.Mask") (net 27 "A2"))
  (pad "25" thru_hole rect (at 10.16 8.89 90) (size 1.6 1.6) (drill 0.8) (layers "*.Cu" "*.Mask") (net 28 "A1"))
  (pad "26" thru_hole rect (at 10.16 11.43 90) (size 1.6 1.6) (drill 0.8) (layers "*.Cu" "*.Mask") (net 29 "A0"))
  (pad "27" thru_hole rect (at 10.16 13.97 90) (size 1.6 1.6) (drill 0.8) (layers "*.Cu" "*.Mask") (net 20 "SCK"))
  (pad "28" thru_hole rect (at 10.16 16.51 90) (size 1.6 1.6) (drill 0.8) (layers "*.Cu" "*.Mask") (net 21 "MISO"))
  (pad "29" thru_hole rect (at 10.16 19.05 90) (size 1.6 1.6) (drill 0.8) (layers "*.Cu" "*.Mask") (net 22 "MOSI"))
  (pad "30" thru_hole rect (at 10.16 21.59 90) (size 1.6 1.6) (drill 0.8) (layers "*.Cu" "*.Mask") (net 23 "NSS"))
  (pad "31" thru_hole rect (at 6.35 5.08 180) (size 1.6 1.6) (drill 0.8) (layers "*.Cu" "*.Mask") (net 14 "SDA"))
  (pad "32" thru_hole rect (at 6.35 2.54 180) (size 1.6 1.6) (drill 0.8) (layers "*.Cu" "*.Mask") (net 13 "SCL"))
  (pad "A6" thru_hole rect (at 3.81 21.59 180) (size 1.6 1.6) (drill 0.8) (layers "*.Cu" "*.Mask"))
  (pad "A7" thru_hole rect (at 6.35 21.59 180) (size 1.6 1.6) (drill 0.8) (layers "*.Cu" "*.Mask"))
  (pad "GND4" thru_hole rect (at 1.27 21.59 180) (size 1.6 1.6) (drill 0.8) (layers "*.Cu" "*.Mask")))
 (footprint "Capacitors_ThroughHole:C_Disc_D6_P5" (layer "F.Cu") (at 70.5 109.5)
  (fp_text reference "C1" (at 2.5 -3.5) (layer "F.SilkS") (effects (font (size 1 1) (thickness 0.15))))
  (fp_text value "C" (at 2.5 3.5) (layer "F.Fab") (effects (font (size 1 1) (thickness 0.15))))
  (pad "1" thru_hole rect (at 0 0) (size 1.4 1.4) (drill 0.9) (layers "*.Cu" "*.Mask" "F.SilkS") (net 3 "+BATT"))
  (pad "2" thru_hole circle (at 5 0) (size 1.4 1.4) (drill 0.9) (layers "*.Cu" "*.Mask" "F.SilkS") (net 1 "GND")))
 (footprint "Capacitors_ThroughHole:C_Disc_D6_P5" (layer "F.Cu") (at 217.5 112.25)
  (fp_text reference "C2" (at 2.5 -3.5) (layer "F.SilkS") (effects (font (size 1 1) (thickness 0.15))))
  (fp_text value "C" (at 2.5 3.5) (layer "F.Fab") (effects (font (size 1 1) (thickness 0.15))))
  (pad "1" thru_hole rect (at 0 0) (size 1.4 1.4) (drill 0.9) (layers "*.Cu" "*.Mask" "F.SilkS") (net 3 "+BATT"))
  (pad "2" thru_hole circle (at 5 0) (size 1.4 1.4) (drill 0.9) (layers "*.Cu" "*.Mask" "F.SilkS") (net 1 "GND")))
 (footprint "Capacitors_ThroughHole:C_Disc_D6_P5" (layer "F.Cu") (at 165 43.5)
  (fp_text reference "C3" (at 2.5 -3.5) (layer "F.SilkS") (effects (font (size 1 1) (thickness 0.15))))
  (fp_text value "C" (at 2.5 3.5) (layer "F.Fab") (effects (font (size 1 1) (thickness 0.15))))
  (pad "1" thru_hole rect (at 0 0) (size 1.4 1.4) (drill 0.9) (layers "*.Cu" "*.Mask" "F.SilkS") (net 3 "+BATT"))
  (pad "2" thru_hole circle (at 5 0) (size 1.4 1.4) (drill 0.9) (layers "*.Cu" "*.Mask" "F.SilkS") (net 1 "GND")))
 (gr_arc (start 101 151) (mid 93.928932 148.071068) (end 91 141) (stroke (width 0.15) (type solid)) (layer "Edge.Cuts"))
 (gr_arc (start 91 141) (mid 93.928932 133.928932) (end 101 131) (stroke (width 0.15) (type solid)) (layer "Edge.Cuts"))
 (gr_arc (start 101 131) (mid 108.071068 133.928932) (end 111 141) (stroke (width 0.15) (type solid)) (layer "Edge.Cuts"))
 (gr_arc (start 172.75 84.75) (mid 165.678932 81.821068) (end 162.75 74.75) (stroke (width 0.15) (type solid)) (layer "Edge.Cuts"))
 (gr_arc (start 162.75 74.75) (mid 165.678932 67.678932) (end 172.75 64.75) (stroke (width 0.15) (type solid)) (layer "Edge.Cuts"))
 (gr_arc (start 101 131) (mid 108.071068 133.928932) (end 111 141) (stroke (width 0.15) (type solid)) (layer "Edge.Cuts"))
 (gr_arc (start 172.75 64.75) (mid 179.821068 67.678932) (end 182.75 74.75) (stroke (width 0.15) (type solid)) (layer "Edge.Cuts"))
 (gr_circle (center 212.75 149.5) (end 214.5 149.5) (stroke (width 0.15) (type solid)) (fill none) (layer "Edge.Cuts"))
 (gr_circle (center 257.75 104.5) (end 259.5 104.5) (stroke (width 0.15) (type solid)) (fill none) (layer "Edge.Cuts"))
 (gr_circle (center 212.75 104.5) (end 214.5 104.5) (stroke (width 0.15) (type solid)) (fill none) (layer "Edge.Cuts"))
 (gr_circle (center 135.25 37.25) (end 137 37.25) (stroke (width 0.15) (type solid)) (fill none) (layer "Edge.Cuts"))
 (gr_circle (center 180.25 37.25) (end 182 37.25) (stroke (width 0.15) (type solid)) (fill none) (layer "Edge.Cuts"))
 (gr_circle (center 135.25 82.25) (end 137 82.25) (stroke (width 0.15) (type solid)) (fill none) (layer "Edge.Cuts"))
 (gr_circle (center 63.5 148.5) (end 65.25 148.5) (stroke (width 0.15) (type solid)) (fill none) (layer "Edge.Cuts"))
 (gr_circle (center 108.5 103.5) (end 110.25 103.5) (stroke (width 0.15) (type solid)) (fill none) (layer "Edge.Cuts"))
 (gr_circle (center 63.5 103.5) (end 65.25 103.5) (stroke (width 0.15) (type solid)) (fill none) (layer "Edge.Cuts"))
 (gr_circle (center 92.25 149.25) (end 93.25 149.25) (stroke (width 0.15) (type solid)) (fill none) (layer "Edge.Cuts"))
 (gr_circle (center 164 83) (end 165 83) (stroke (width 0.15) (type solid)) (fill none) (layer "Edge.Cuts"))
 (gr_circle (center 241.5 150.25) (end 242.5 150.25) (stroke (width 0.15) (type solid)) (fill none) (layer "Edge.Cuts"))
 (gr_circle (center 258.5 133.25) (end 259.5 133.25) (stroke (width 0.15) (type solid)) (fill none) (layer "Edge.Cuts"))
 (gr_circle (center 181 66) (end 182 66) (stroke (width 0.15) (type solid)) (fill none) (layer "Edge.Cuts"))
 (gr_circle (center 109.25 132.25) (end 110.25 132.25) (stroke (width 0.15) (type solid)) (fill none) (layer "Edge.Cuts"))
 (gr_arc (start 240.25 142) (mid 243.178932 134.928932) (end 250.25 132) (stroke (width 0.15) (type solid)) (layer "Edge.Cuts"))
 (gr_line (start 132.75 34.75) (end 132.75 84.25) (stroke (width 0.15) (type solid)) (layer "Edge.Cuts"))
 (gr_circle (center 140 174.25) (end 141 174.25) (stroke (width 0.15) (type solid)) (fill none) (layer "Edge.Cuts"))
 (gr_line (start 210.25 152) (end 210.25 102) (stroke (width 0.15) (type solid)) (layer "Edge.Cuts"))
 (gr_line (start 132.75 84.75) (end 132.75 84.25) (stroke (width 0.15) (type solid)) (layer "Edge.Cuts"))
 (gr_arc (start 250.25 132) (mid 257.321068 134.928932) (end 260.25 142) (stroke (width 0.15) (type solid)) (layer "Edge.Cuts"))
 (gr_line (start 250.25 152) (end 210.25 152) (stroke (width 0.15) (type solid)) (layer "Edge.Cuts"))
 (gr_line (start 210.25 102) (end 260.25 102) (stroke (width 0.15) (type solid)) (layer "Edge.Cuts"))
 (gr_line (start 182.75 34.75) (end 132.75 34.75) (stroke (width 0.15) (type solid)) (layer "Edge.Cuts"))
 (gr_line (start 61 101) (end 111 101) (stroke (width 0.15) (type solid)) (layer "Edge.Cuts"))
 (gr_line (start 111 101) (end 111 141) (stroke (width 0.15) (type solid)) (layer "Edge.Cuts"))
 (gr_circle (center 128 173.5) (end 129.75 173.5) (stroke (width 0.15) (type solid)) (fill none) (layer "Edge.Cuts"))
 (gr_line (start 182.75 74.75) (end 182.75 34.75) (stroke (width 0.15) (type solid)) (layer "Edge.Cuts"))
 (gr_line (start 101 151) (end 61 151) (stroke (width 0.15) (type solid)) (layer "Edge.Cuts"))
 (gr_arc (start 250.25 152) (mid 243.178932 149.071068) (end 240.25 142) (stroke (width 0.15) (type solid)) (layer "Edge.Cuts"))
 (gr_line (start 61 151) (end 61 101) (stroke (width 0.15) (type solid)) (layer "Edge.Cuts"))
 (gr_line (start 172.75 84.75) (end 132.75 84.75) (stroke (width 0.15) (type solid)) (layer "Edge.Cuts"))
 (gr_line (start 260.25 142) (end 260.25 102) (stroke (width 0.15) (type solid)) (layer "Edge.Cuts"))
 (segment (start 156.75 49.75) (end 156 49.75) (width 0.25) (layer "F.Cu") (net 1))
 (segment (start 154.75 48.5) (end 154.75 40.75) (width 0.25) (layer "F.Cu") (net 1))
 (segment (start 156 49.75) (end 154.75 48.5) (width 0.25) (layer "F.Cu") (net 1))
 (segment (start 175.42 37.1524) (end 175.42 37) (width 0.25) (layer "F.Cu") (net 15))
 (segment (start 136.266 67.26) (end 135 67.26) (width 0.25) (layer "F.Cu") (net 20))
 (segment (start 135 77.42) (end 135.1524 77.42) (width 0.25) (layer "F.Cu") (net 24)))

